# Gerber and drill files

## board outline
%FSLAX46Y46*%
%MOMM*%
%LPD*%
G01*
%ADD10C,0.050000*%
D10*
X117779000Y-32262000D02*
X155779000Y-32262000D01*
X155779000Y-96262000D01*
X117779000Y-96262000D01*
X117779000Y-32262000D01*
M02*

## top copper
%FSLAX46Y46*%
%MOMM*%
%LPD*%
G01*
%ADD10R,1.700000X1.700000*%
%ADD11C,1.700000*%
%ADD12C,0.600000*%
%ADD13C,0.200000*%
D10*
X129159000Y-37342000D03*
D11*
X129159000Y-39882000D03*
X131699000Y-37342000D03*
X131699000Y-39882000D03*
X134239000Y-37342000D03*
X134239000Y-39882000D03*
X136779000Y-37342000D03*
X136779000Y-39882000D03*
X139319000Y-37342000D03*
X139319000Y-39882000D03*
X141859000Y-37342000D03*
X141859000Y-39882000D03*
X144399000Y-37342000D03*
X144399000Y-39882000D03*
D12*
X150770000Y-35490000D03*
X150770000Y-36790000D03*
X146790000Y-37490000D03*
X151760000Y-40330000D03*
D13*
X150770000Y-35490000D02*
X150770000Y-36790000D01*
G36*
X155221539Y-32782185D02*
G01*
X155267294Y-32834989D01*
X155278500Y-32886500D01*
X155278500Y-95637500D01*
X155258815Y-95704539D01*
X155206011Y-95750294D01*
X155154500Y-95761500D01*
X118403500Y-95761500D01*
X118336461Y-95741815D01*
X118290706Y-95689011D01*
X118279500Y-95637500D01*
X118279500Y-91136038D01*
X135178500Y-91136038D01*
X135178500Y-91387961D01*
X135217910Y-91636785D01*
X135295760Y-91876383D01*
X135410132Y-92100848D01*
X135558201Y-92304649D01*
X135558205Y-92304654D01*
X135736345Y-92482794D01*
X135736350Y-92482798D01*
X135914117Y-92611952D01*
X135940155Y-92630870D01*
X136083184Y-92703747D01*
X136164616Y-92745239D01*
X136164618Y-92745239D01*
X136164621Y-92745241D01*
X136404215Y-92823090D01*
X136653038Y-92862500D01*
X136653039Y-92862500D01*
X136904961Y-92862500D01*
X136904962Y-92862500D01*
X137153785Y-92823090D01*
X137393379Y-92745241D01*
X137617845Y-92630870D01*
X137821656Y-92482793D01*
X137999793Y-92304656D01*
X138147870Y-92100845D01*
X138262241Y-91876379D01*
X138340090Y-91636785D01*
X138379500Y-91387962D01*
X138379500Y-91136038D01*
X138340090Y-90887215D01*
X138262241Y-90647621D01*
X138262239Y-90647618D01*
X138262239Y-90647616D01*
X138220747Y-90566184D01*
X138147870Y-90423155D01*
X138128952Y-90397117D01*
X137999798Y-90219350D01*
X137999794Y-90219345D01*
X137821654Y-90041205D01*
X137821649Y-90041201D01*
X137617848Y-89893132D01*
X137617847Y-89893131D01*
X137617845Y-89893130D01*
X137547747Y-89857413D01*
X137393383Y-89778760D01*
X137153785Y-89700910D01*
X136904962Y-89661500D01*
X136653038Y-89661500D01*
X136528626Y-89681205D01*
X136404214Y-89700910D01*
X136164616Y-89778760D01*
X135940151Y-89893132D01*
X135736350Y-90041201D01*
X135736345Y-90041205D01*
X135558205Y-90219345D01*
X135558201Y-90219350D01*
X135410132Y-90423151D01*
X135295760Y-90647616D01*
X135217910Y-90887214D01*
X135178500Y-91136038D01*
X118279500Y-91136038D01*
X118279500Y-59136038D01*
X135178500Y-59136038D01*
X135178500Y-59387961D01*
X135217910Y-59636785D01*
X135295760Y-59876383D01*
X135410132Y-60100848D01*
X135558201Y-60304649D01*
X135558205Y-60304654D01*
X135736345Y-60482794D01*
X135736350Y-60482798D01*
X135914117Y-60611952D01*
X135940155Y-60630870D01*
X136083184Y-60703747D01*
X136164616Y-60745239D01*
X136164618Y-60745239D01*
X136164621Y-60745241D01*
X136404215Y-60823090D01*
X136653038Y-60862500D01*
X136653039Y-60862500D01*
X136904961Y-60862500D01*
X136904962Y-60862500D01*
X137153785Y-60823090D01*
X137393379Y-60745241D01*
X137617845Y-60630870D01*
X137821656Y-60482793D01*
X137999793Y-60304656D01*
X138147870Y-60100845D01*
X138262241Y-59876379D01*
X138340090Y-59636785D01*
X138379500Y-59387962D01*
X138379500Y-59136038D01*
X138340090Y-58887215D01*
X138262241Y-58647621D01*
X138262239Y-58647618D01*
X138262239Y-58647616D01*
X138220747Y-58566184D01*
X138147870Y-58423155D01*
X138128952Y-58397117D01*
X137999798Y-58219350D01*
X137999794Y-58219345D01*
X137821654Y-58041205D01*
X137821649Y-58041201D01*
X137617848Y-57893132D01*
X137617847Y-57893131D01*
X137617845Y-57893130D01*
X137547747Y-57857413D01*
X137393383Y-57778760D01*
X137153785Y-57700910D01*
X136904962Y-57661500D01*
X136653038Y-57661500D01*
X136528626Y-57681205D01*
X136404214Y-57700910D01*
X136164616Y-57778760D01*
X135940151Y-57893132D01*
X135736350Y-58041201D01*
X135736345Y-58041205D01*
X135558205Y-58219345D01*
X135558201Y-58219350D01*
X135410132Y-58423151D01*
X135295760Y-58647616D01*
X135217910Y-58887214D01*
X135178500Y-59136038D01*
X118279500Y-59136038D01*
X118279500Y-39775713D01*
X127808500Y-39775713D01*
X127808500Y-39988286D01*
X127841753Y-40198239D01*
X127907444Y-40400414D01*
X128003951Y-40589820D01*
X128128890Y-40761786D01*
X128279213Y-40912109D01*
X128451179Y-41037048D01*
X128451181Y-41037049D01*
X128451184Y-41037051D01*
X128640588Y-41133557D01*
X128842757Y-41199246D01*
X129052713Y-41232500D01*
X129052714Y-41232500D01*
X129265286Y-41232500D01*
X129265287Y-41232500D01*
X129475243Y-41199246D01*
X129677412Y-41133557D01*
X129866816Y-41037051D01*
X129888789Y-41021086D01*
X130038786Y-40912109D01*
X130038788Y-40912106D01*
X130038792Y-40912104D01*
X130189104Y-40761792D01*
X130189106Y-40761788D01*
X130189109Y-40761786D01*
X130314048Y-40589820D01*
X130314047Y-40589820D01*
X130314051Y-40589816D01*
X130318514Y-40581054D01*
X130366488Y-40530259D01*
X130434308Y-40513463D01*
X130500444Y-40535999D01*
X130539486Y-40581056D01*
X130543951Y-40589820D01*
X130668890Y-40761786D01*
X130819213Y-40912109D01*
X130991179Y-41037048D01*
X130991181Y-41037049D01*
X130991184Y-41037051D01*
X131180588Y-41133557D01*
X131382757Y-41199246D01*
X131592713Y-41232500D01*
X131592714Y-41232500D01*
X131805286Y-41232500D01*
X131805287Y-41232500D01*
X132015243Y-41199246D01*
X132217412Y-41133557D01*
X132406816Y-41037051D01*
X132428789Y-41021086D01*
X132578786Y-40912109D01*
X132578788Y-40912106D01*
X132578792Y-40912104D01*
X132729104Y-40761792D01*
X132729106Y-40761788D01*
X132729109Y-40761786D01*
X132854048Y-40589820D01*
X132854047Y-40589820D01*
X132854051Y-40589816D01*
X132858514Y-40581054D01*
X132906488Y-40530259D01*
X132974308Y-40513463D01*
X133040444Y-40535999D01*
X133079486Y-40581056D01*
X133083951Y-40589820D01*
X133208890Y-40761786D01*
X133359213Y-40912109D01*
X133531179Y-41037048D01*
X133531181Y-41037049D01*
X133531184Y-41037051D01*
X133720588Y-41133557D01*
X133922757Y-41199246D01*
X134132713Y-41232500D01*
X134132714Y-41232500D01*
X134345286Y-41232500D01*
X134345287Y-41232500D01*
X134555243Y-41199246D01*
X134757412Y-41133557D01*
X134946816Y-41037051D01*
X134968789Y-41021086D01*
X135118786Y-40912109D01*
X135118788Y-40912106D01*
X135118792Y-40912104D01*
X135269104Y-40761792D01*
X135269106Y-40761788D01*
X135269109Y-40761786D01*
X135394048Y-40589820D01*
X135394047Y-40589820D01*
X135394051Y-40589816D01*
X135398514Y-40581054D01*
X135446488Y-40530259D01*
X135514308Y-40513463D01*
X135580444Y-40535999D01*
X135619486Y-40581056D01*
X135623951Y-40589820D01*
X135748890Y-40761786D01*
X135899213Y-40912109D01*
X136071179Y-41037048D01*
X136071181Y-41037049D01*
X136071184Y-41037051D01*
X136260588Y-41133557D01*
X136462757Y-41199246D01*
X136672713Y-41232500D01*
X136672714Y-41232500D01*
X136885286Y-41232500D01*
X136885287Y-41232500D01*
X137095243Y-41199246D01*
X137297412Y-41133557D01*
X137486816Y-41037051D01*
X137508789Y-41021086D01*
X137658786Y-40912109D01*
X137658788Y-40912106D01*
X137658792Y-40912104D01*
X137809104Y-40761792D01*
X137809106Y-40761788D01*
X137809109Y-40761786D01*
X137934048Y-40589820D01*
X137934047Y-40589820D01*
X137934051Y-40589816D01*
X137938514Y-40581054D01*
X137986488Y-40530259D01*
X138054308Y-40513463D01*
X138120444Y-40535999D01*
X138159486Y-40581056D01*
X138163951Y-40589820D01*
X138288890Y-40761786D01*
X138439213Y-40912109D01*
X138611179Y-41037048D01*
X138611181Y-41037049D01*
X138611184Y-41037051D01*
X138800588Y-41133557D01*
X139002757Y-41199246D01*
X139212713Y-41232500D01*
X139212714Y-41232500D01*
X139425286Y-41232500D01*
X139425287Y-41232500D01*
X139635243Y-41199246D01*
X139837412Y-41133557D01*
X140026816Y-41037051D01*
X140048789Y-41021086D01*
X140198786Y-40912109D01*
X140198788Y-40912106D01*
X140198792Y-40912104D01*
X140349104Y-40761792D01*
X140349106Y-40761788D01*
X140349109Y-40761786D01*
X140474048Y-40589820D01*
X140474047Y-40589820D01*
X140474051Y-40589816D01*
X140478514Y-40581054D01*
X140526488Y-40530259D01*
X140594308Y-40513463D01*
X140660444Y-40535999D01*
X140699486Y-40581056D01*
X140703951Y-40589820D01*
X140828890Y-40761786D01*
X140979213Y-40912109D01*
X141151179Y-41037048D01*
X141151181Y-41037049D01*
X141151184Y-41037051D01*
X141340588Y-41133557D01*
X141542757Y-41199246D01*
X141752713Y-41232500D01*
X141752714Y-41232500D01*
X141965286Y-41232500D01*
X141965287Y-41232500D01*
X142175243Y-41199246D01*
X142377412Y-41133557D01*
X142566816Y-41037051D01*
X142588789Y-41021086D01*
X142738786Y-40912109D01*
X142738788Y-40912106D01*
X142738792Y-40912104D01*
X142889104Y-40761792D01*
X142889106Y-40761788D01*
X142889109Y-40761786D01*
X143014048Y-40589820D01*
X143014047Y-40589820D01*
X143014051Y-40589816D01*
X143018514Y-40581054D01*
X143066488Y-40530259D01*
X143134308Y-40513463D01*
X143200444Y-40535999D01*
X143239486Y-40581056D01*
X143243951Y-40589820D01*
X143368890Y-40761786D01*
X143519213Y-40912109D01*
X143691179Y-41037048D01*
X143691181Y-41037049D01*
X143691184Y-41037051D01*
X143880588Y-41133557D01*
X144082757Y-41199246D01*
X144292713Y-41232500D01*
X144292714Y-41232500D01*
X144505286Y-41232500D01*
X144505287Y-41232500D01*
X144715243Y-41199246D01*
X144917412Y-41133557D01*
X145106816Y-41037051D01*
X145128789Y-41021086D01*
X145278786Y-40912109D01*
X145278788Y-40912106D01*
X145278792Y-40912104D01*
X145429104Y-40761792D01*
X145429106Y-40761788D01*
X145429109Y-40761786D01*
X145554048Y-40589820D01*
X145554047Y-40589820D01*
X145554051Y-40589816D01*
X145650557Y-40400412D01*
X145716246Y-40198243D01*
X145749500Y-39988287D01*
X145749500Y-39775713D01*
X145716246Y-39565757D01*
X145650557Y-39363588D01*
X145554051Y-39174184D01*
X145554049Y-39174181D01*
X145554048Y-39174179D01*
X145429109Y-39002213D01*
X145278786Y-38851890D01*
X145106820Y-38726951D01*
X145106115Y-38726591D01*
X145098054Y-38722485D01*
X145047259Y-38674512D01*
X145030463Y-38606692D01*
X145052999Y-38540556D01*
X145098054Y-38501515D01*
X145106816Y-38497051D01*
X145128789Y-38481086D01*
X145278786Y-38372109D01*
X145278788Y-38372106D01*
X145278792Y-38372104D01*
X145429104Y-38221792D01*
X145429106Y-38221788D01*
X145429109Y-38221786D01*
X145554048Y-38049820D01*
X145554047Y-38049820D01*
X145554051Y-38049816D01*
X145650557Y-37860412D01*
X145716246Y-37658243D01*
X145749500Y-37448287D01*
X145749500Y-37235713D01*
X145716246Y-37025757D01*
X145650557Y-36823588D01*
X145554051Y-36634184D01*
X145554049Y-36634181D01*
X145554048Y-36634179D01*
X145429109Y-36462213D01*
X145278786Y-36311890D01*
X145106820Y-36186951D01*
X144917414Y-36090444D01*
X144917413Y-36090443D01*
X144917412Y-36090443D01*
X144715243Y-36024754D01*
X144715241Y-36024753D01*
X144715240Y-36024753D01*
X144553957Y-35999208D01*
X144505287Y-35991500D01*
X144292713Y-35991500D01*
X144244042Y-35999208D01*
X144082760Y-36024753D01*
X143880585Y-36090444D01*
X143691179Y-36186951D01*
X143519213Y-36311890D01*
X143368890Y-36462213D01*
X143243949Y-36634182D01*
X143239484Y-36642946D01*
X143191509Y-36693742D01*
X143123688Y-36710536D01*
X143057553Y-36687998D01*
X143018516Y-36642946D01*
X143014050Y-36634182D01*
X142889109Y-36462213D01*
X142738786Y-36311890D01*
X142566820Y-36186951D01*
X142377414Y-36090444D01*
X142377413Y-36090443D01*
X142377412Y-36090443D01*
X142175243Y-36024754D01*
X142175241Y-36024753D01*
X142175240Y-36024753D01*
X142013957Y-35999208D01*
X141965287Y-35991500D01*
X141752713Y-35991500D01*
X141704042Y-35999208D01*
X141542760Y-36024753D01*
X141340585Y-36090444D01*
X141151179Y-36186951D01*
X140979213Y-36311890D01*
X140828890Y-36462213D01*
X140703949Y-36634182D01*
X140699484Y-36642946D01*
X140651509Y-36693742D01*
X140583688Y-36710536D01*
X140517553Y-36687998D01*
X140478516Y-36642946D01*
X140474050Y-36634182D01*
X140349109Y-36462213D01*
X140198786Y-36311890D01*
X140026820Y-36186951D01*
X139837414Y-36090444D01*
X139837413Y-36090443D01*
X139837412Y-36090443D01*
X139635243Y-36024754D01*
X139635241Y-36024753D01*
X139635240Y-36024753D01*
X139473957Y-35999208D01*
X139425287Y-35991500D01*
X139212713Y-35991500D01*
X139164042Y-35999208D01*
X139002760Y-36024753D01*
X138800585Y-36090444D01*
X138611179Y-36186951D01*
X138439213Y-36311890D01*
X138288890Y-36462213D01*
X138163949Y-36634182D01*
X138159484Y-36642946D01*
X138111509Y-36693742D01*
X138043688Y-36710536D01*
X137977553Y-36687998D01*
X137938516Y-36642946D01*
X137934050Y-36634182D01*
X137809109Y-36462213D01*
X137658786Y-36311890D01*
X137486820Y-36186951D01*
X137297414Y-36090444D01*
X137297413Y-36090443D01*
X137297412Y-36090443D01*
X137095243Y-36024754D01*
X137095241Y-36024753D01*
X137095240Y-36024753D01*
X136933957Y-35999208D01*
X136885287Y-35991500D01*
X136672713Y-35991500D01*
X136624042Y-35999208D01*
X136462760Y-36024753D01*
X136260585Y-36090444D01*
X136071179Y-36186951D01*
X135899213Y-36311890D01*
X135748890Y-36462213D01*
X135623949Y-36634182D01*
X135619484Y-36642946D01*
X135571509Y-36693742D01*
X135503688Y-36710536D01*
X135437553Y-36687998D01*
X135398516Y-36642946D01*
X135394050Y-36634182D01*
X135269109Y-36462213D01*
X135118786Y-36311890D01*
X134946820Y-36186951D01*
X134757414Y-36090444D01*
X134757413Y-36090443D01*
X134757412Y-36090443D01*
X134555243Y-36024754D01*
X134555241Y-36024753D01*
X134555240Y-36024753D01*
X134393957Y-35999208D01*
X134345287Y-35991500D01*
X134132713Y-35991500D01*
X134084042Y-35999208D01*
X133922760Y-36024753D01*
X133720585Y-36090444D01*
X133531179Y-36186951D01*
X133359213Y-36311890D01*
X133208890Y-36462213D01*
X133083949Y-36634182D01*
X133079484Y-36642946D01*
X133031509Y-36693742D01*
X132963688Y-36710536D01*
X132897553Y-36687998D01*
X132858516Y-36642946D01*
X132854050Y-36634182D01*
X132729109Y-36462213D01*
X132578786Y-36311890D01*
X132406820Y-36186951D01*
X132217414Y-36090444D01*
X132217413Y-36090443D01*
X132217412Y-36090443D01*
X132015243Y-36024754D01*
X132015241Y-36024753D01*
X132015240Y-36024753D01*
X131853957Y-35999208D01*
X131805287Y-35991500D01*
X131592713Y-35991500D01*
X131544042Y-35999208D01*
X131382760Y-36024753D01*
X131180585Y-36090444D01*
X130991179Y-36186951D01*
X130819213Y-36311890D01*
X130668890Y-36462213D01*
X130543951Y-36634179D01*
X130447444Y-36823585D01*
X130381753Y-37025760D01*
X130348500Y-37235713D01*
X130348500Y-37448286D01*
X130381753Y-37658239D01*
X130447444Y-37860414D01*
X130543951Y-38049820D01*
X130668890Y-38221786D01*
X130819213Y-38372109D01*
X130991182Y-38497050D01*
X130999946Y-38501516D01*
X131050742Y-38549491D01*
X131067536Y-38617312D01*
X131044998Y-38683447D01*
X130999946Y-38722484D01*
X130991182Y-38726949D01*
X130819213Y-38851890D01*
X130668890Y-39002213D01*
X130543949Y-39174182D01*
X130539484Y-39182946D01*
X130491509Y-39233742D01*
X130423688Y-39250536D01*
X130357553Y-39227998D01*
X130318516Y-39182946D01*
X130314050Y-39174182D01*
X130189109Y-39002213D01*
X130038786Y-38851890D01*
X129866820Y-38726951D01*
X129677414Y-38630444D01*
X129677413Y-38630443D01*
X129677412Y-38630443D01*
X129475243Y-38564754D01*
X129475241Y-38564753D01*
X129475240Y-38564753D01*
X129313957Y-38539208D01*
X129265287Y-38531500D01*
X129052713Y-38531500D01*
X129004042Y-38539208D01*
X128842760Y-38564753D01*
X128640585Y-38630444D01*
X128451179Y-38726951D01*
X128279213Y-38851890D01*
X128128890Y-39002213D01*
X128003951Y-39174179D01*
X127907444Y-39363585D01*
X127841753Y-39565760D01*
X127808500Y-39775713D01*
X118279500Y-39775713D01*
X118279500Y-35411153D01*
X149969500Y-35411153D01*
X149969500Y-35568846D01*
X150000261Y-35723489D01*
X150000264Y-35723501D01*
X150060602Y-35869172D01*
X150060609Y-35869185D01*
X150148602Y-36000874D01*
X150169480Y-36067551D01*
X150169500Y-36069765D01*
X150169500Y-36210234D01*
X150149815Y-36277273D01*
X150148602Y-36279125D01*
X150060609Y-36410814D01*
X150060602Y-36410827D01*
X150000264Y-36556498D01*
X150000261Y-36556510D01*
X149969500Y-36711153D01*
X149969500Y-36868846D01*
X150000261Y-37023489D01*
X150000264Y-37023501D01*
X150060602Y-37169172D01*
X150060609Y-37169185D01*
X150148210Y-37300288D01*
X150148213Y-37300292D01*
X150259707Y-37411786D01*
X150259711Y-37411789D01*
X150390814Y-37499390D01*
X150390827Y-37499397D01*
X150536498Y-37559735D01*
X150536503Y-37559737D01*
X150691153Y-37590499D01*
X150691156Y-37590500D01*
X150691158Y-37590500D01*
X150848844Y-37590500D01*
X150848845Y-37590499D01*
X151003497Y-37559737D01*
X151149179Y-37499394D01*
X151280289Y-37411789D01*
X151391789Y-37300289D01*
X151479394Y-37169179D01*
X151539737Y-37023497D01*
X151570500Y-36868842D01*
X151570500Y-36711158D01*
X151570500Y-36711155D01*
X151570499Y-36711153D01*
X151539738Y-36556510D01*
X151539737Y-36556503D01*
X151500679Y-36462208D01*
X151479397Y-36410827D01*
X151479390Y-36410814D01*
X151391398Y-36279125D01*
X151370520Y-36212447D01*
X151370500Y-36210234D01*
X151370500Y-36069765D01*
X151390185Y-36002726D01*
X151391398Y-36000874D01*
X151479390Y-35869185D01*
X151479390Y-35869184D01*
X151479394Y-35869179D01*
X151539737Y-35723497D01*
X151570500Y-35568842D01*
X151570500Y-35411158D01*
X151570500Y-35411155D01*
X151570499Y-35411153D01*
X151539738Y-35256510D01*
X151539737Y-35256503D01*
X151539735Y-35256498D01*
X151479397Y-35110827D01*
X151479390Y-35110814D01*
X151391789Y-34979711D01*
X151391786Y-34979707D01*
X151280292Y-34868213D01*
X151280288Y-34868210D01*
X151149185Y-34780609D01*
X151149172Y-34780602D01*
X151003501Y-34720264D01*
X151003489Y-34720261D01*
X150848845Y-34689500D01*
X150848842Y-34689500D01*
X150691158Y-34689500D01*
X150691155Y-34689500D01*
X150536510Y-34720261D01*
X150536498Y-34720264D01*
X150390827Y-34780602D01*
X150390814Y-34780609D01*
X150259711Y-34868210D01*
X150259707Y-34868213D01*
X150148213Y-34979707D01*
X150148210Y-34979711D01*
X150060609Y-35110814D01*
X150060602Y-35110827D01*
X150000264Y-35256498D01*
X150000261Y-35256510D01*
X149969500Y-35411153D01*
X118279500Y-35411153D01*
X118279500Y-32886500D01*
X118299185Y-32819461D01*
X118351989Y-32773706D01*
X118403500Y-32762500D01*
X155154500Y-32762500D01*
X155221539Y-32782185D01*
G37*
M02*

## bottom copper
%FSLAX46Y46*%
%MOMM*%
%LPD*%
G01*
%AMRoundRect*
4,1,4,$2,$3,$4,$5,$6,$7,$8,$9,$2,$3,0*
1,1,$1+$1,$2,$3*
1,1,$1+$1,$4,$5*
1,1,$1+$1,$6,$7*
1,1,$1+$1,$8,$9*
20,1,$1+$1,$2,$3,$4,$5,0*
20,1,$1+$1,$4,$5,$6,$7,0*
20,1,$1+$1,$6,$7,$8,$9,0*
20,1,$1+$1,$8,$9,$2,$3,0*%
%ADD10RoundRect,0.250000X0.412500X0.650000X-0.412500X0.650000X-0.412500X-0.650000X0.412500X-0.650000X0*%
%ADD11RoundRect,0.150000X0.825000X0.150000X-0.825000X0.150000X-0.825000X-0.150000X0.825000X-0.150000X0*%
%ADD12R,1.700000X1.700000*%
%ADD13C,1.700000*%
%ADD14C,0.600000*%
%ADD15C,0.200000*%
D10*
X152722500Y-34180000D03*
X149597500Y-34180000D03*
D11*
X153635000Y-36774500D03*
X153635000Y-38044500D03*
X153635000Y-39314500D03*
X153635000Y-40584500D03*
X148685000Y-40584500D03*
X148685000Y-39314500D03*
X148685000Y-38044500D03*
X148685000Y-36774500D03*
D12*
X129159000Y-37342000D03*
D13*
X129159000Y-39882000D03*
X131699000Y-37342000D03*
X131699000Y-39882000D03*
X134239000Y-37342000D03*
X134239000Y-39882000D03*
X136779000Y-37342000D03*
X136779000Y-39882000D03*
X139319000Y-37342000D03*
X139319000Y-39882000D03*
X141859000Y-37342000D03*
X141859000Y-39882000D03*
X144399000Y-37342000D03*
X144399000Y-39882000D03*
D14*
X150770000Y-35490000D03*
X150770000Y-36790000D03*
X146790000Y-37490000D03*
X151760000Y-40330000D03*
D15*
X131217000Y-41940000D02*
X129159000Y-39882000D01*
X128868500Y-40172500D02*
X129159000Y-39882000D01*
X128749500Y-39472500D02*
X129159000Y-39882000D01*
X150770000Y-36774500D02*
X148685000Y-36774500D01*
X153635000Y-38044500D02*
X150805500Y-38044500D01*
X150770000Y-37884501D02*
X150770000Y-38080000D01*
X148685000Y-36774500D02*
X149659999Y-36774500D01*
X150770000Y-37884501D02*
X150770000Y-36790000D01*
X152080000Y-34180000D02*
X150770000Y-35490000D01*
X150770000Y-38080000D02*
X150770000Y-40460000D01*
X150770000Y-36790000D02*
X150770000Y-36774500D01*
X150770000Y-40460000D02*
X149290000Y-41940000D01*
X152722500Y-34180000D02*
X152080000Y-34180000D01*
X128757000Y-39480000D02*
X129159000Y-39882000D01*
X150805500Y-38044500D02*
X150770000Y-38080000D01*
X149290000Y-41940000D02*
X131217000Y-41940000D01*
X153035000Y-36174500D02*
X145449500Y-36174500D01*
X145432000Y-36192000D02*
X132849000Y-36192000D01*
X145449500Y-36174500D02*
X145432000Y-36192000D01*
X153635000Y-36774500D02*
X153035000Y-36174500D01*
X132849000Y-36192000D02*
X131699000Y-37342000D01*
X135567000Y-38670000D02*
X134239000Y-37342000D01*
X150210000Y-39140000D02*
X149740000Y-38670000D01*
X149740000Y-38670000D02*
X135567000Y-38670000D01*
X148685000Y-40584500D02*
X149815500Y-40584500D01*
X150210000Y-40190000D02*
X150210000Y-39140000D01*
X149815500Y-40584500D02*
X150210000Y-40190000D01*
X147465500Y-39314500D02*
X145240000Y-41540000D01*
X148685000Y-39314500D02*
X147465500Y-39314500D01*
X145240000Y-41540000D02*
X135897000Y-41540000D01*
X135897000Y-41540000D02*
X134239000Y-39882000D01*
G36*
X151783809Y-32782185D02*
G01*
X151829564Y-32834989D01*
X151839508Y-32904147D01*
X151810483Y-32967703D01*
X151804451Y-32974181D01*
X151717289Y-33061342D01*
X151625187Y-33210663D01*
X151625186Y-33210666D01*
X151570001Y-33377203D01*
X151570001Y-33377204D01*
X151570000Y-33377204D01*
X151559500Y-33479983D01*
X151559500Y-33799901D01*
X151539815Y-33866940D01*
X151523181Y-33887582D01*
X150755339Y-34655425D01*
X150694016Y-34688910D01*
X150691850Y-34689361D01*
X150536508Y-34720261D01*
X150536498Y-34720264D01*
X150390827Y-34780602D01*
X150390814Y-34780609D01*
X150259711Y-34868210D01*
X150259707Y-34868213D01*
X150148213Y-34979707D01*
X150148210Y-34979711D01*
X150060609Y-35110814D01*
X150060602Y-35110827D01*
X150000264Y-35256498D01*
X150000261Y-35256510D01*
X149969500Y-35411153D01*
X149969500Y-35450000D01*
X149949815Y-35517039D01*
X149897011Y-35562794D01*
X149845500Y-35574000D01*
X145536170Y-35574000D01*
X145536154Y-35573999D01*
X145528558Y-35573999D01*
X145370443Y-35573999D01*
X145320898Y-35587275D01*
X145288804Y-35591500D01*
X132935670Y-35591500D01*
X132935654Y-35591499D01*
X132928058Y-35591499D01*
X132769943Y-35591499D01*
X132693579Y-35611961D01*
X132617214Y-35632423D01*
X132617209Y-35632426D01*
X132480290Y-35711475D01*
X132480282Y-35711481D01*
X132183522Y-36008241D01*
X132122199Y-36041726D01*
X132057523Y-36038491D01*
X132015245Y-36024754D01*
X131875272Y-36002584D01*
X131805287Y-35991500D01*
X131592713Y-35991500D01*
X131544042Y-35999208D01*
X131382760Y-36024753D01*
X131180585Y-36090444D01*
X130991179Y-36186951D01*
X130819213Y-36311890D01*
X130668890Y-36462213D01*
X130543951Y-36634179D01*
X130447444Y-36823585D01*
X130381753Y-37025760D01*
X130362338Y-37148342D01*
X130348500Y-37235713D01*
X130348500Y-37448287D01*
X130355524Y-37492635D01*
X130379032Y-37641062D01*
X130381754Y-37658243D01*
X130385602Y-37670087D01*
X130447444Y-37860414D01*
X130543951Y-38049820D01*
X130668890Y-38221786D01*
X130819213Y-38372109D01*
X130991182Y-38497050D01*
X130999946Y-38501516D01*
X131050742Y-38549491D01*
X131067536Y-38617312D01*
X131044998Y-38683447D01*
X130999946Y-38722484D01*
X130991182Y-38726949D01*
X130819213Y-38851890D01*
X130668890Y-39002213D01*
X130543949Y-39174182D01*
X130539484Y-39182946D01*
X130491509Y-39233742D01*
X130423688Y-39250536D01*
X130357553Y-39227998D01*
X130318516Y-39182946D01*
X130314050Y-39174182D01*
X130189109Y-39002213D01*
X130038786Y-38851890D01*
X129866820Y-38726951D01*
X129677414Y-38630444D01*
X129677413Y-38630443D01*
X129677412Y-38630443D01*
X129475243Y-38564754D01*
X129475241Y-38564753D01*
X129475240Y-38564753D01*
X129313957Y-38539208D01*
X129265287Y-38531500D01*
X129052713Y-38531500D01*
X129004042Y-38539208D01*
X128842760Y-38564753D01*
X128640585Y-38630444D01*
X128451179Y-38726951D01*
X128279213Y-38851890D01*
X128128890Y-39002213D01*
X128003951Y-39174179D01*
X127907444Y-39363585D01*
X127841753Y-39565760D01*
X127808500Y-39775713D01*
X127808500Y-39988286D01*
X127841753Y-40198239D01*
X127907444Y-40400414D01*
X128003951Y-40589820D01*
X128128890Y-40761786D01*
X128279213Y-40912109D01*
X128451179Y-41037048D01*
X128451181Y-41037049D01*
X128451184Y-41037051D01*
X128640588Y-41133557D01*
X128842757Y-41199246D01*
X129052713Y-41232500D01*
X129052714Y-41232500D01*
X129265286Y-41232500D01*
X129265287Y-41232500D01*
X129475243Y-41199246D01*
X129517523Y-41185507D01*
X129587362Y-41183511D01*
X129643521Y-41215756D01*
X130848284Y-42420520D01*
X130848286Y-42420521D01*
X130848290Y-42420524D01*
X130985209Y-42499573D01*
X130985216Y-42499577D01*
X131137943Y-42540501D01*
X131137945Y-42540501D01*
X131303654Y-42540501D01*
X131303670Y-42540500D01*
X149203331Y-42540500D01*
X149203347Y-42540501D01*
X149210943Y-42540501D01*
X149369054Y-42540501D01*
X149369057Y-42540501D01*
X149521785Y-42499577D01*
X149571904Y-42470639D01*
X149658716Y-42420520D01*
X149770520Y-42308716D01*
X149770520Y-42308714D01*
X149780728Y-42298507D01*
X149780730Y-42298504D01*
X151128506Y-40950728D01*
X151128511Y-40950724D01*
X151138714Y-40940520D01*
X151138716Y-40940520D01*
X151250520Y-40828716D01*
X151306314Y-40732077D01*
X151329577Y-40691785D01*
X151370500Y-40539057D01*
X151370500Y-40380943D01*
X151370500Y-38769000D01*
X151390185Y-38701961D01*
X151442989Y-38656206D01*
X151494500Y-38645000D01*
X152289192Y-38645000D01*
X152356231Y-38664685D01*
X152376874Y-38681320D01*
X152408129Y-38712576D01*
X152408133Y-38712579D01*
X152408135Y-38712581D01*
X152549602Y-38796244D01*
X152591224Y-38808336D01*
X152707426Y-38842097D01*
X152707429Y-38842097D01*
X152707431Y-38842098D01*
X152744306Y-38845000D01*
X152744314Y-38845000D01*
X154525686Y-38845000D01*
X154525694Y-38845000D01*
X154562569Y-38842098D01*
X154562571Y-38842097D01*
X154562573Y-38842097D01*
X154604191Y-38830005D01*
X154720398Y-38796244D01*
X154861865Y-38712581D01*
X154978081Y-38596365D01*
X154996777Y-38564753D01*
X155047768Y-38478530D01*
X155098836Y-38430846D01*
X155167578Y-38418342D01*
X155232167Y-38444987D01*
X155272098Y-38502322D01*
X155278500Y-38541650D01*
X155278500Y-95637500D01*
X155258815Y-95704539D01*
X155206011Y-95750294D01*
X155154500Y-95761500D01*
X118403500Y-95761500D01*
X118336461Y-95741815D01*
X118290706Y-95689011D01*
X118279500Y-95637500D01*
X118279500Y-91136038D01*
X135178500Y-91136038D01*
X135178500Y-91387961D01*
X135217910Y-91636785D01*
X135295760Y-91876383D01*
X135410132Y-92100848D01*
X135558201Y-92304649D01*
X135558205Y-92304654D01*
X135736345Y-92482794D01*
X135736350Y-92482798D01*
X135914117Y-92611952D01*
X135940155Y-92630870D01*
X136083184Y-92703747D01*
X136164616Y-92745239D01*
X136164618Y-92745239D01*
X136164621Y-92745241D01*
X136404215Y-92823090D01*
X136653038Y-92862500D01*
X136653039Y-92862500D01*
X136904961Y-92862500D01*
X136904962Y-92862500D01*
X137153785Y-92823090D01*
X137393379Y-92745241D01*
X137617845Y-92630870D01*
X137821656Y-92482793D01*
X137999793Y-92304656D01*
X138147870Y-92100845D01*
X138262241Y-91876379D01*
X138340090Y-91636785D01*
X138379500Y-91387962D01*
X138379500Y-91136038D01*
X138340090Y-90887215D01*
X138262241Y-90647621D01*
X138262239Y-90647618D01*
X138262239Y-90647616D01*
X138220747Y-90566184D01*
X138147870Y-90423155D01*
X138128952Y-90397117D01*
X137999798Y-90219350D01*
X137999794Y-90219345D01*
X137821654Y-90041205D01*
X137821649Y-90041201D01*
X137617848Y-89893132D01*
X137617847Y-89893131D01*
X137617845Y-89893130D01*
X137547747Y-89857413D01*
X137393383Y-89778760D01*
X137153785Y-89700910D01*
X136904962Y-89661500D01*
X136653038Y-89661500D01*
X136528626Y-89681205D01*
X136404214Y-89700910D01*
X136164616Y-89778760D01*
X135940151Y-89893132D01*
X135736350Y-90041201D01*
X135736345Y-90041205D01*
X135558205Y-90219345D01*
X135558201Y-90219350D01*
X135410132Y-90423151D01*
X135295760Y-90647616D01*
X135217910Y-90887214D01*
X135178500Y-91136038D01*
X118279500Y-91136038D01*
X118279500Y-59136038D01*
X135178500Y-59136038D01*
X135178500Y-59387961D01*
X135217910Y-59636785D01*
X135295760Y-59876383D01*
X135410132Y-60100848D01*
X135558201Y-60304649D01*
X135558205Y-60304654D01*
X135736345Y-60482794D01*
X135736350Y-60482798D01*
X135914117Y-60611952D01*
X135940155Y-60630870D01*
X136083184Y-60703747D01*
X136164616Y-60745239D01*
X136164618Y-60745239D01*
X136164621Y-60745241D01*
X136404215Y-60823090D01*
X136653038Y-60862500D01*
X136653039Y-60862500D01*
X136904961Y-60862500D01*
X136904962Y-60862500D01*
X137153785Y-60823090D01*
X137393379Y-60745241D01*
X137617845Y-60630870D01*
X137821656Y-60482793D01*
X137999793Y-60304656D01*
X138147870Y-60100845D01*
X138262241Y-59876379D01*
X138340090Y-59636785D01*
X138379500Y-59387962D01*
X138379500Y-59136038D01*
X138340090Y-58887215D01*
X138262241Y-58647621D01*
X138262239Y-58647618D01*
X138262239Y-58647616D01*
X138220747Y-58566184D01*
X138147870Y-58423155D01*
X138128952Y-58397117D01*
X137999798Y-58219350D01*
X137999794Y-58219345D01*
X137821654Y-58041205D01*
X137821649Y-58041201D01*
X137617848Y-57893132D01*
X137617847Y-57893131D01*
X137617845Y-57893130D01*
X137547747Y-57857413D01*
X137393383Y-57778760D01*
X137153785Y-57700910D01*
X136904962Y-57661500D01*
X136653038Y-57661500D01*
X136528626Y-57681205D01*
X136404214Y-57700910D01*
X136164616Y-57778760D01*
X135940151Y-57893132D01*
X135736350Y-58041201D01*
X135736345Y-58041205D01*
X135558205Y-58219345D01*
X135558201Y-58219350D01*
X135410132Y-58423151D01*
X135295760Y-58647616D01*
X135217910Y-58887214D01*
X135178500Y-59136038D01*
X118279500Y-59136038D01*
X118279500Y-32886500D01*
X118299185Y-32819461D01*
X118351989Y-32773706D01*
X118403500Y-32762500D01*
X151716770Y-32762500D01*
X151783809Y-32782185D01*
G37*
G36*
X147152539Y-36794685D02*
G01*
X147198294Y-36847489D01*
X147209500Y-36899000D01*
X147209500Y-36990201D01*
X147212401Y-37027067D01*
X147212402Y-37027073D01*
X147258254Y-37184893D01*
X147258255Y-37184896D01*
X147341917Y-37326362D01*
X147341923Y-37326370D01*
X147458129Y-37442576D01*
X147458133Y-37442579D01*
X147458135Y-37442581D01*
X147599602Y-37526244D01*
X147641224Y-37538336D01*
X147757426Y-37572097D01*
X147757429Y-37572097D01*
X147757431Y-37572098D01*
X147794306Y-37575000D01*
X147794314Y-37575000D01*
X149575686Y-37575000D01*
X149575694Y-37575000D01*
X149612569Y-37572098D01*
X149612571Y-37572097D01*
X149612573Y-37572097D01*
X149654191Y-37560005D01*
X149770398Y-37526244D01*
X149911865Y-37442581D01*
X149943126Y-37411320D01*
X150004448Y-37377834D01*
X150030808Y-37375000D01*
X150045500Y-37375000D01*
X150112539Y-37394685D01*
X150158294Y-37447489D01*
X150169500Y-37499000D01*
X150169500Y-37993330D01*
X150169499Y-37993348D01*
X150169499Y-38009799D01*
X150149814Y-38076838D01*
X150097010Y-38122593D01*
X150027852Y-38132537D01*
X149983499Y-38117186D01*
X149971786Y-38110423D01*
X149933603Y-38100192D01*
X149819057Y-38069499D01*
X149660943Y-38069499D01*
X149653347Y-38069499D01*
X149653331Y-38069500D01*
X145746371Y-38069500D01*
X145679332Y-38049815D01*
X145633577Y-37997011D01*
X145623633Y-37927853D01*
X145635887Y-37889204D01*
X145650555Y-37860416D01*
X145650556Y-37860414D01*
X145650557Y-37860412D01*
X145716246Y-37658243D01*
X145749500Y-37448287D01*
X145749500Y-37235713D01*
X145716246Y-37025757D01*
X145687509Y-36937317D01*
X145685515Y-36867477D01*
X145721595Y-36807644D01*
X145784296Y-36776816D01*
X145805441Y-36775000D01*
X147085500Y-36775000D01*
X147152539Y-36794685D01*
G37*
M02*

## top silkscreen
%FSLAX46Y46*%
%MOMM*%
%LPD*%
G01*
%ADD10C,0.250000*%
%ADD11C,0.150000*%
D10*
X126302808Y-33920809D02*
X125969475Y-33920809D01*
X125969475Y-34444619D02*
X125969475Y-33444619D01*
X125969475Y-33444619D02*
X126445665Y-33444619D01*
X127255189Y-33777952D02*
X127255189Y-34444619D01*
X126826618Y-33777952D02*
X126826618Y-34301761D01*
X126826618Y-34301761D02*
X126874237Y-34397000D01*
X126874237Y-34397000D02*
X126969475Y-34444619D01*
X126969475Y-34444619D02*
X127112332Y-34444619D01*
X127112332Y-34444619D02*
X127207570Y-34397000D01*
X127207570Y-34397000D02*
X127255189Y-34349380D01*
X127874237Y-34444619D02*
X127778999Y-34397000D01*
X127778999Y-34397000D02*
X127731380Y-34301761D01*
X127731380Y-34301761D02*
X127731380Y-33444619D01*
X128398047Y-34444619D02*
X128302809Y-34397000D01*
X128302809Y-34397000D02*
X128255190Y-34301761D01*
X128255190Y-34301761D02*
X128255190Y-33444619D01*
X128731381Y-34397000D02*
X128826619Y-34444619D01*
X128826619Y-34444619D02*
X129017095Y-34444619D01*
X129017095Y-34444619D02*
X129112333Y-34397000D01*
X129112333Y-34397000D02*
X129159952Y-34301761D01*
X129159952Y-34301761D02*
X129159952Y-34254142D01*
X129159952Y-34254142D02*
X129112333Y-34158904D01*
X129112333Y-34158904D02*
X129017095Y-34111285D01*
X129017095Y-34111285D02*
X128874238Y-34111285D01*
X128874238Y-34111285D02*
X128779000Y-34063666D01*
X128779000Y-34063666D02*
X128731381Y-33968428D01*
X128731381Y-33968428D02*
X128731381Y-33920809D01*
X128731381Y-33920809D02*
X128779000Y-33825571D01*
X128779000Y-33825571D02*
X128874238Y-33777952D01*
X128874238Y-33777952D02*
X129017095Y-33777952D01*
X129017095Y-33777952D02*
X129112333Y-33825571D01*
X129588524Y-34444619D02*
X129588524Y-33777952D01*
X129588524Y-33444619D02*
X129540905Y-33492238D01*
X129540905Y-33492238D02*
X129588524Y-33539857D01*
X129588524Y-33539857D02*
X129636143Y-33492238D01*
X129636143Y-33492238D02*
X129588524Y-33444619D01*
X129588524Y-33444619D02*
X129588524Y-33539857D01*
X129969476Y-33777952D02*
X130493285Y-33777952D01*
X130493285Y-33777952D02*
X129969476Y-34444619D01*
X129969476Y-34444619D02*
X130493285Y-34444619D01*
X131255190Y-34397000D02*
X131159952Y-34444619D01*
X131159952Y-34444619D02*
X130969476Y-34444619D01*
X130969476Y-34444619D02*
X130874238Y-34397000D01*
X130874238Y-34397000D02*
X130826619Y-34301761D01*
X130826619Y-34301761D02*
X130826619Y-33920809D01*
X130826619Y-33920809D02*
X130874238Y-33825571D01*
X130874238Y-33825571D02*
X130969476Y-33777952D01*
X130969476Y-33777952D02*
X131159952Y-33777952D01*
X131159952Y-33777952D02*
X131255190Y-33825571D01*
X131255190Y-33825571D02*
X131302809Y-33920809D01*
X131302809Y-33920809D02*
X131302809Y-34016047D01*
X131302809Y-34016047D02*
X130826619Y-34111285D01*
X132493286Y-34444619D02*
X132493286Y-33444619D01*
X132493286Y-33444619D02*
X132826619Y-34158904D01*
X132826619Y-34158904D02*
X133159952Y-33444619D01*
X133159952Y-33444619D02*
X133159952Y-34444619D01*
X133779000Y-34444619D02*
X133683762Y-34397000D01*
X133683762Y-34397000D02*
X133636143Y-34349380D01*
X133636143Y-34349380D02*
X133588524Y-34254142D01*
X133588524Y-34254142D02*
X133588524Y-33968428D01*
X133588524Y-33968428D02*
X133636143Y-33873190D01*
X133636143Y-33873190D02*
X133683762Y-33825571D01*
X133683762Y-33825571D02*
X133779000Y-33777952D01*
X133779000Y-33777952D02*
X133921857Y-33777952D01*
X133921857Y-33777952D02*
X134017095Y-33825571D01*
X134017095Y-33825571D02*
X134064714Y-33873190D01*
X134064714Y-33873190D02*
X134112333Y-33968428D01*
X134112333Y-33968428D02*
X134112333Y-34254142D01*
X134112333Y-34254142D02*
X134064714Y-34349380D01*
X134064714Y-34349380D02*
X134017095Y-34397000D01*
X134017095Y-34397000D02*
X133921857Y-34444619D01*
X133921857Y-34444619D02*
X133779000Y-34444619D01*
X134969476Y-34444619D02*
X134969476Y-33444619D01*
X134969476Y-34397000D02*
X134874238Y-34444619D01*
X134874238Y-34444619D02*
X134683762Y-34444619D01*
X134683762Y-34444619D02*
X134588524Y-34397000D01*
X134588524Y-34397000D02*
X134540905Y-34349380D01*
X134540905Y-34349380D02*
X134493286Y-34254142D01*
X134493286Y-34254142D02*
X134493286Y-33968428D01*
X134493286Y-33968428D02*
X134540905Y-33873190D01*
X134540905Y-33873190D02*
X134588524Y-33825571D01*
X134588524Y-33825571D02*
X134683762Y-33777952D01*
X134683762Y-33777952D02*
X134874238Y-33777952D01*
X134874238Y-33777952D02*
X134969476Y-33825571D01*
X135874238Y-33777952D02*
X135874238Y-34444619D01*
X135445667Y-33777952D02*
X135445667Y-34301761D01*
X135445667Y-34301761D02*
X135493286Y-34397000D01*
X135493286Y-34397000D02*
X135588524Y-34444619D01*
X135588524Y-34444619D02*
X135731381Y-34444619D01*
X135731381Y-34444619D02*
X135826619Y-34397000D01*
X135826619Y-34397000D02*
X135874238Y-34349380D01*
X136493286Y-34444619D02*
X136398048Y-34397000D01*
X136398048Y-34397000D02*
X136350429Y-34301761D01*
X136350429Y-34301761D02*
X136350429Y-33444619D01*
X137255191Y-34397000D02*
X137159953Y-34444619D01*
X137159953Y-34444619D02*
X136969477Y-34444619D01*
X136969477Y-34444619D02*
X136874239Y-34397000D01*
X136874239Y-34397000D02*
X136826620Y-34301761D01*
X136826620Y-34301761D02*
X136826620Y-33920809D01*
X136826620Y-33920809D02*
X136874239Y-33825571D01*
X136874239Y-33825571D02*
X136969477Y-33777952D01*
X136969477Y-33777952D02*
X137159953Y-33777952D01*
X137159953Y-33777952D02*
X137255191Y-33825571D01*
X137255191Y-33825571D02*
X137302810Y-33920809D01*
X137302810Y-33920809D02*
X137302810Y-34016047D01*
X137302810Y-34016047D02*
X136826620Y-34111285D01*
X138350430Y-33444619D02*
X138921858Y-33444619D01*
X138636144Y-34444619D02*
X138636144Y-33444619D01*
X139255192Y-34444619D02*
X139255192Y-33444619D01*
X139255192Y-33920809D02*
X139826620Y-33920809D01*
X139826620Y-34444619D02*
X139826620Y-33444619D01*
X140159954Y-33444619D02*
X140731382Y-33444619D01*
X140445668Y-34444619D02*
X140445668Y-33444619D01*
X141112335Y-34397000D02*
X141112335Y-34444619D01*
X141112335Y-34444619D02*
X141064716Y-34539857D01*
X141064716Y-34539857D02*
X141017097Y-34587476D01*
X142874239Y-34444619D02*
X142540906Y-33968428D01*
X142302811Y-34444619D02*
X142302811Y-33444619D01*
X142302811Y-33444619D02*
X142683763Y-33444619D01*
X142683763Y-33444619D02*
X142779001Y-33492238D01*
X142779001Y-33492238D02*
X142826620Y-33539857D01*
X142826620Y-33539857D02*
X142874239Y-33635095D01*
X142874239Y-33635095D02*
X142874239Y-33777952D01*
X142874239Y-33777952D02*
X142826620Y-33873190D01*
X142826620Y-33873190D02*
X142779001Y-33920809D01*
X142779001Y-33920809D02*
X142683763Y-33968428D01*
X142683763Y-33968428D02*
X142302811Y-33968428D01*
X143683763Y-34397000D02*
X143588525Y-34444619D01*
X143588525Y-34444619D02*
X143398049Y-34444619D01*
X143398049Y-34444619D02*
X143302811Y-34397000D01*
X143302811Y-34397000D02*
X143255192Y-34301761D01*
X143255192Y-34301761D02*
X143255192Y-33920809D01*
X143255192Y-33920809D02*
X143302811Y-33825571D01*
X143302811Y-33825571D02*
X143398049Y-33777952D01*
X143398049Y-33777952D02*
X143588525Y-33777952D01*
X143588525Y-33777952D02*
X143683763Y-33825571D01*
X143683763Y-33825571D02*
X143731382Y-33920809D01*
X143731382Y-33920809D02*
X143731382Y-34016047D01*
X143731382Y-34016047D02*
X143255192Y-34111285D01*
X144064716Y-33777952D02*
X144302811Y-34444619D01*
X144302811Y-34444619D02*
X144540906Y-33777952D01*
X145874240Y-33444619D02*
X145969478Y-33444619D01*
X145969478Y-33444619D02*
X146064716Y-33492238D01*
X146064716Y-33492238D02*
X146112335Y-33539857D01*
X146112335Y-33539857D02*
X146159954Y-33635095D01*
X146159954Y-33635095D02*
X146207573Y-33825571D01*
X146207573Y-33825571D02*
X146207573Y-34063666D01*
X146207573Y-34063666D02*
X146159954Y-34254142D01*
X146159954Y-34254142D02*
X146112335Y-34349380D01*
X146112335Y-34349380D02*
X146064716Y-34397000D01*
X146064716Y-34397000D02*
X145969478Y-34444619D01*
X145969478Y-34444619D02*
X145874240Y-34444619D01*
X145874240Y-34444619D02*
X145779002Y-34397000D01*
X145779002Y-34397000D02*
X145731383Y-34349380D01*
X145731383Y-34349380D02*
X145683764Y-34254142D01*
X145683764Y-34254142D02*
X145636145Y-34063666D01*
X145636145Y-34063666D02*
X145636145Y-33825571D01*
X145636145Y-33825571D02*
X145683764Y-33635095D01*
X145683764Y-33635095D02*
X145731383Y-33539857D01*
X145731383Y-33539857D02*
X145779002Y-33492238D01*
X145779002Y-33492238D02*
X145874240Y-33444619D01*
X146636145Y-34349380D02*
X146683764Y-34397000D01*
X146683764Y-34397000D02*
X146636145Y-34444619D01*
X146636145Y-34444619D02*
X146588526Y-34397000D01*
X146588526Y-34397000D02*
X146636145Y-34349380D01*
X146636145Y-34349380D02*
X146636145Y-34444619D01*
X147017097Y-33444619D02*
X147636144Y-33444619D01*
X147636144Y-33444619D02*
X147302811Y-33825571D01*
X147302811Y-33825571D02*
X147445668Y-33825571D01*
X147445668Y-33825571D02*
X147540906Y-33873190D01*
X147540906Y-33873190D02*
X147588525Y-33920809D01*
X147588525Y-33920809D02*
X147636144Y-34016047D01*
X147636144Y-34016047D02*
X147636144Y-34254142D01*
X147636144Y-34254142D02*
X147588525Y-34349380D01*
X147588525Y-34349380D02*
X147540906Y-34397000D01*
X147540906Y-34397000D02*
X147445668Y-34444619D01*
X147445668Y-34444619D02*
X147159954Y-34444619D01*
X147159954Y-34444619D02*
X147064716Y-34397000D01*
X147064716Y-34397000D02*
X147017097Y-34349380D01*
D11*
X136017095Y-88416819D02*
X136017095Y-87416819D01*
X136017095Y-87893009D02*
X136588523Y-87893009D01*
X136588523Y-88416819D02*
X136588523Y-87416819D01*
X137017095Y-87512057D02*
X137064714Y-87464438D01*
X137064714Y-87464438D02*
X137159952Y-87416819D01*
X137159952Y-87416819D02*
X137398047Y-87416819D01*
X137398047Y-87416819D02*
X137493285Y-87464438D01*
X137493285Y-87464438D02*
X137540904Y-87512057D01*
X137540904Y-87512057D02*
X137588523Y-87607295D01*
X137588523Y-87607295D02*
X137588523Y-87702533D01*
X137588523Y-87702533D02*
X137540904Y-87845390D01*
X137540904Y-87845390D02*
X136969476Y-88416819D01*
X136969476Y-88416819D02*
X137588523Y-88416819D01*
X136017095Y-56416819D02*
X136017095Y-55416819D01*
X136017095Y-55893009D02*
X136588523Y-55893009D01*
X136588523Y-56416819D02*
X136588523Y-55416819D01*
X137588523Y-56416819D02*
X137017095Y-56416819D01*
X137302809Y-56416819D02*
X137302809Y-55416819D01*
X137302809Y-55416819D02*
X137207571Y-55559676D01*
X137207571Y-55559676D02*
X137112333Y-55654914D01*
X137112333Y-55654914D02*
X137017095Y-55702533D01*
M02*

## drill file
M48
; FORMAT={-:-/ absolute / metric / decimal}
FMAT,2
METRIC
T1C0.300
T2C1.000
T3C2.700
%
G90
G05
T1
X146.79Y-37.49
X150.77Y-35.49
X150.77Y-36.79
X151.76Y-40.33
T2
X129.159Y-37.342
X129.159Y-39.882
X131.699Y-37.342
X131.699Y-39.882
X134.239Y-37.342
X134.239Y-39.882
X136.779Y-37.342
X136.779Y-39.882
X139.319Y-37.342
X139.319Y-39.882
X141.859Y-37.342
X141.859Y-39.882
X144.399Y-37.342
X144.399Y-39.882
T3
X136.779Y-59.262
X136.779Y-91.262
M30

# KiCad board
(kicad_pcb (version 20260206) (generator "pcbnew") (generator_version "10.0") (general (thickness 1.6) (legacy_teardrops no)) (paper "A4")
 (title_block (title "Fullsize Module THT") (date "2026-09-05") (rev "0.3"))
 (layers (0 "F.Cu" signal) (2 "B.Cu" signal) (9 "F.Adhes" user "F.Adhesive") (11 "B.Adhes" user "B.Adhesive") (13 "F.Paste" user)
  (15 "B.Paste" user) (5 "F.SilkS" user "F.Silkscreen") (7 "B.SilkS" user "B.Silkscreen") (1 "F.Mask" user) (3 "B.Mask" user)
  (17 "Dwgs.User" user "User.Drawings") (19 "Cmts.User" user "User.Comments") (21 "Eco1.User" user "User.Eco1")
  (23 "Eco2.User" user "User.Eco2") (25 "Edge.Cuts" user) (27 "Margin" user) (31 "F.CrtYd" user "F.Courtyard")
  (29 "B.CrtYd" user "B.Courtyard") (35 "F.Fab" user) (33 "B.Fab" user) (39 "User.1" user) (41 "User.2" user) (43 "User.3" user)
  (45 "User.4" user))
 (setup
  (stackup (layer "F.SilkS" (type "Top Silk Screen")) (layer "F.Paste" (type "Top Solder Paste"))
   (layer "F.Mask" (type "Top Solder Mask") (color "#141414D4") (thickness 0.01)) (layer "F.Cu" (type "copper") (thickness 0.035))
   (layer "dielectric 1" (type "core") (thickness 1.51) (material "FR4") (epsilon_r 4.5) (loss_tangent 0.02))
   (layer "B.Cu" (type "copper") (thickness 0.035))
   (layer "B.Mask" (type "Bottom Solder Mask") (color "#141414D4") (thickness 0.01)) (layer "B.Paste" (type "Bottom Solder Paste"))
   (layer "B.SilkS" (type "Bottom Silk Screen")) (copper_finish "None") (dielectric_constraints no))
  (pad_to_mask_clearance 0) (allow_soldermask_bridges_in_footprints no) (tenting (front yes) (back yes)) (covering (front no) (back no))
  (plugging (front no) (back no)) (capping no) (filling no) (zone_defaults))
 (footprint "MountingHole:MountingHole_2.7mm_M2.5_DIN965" (layer "F.Cu") (at 136.779 91.262)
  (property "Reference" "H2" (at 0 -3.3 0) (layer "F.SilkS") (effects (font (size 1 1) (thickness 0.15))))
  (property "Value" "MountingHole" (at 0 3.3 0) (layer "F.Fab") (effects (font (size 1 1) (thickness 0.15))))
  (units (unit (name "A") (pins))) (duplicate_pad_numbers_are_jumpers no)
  (pad "" np_thru_hole circle (at 0 0) (size 2.7 2.7) (drill 2.7) (layers "*.Cu" "*.Mask")))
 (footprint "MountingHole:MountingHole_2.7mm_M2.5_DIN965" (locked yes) (layer "F.Cu") (at 136.779 59.262)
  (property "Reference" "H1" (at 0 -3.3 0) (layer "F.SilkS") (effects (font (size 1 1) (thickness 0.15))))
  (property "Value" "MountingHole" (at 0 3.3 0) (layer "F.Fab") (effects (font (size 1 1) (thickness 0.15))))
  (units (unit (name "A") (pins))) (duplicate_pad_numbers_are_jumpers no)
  (pad "" np_thru_hole circle (at 0 0) (size 2.7 2.7) (drill 2.7) (layers "*.Cu" "*.Mask")))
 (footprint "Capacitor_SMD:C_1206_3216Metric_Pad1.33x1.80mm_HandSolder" (layer "B.Cu") (at 151.16 34.18 180)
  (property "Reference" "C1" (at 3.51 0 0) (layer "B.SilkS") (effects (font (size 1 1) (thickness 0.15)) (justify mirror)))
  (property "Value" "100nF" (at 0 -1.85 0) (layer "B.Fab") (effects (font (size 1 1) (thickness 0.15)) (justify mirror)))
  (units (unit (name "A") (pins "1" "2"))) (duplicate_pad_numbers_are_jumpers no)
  (pad "1" smd roundrect (at -1.5625 0 180) (size 1.325 1.8) (layers "B.Cu" "B.Mask" "B.Paste") (roundrect_rratio 0.188679) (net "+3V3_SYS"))
  (pad "2" smd roundrect (at 1.5625 0 180) (size 1.325 1.8) (layers "B.Cu" "B.Mask" "B.Paste") (roundrect_rratio 0.188679) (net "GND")
   (zone_connect 2)))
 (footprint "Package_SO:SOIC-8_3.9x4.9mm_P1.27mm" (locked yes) (layer "B.Cu") (at 151.16 38.6795 180)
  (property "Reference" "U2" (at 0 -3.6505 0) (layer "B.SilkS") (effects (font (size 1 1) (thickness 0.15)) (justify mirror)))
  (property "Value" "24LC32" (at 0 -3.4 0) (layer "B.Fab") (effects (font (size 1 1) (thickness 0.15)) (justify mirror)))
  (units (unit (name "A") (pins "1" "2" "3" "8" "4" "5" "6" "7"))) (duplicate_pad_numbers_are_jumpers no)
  (pad "1" smd roundrect (at -2.475 1.905 180) (size 1.95 0.6) (layers "B.Cu" "B.Mask" "B.Paste") (roundrect_rratio 0.25) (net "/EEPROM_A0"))
  (pad "2" smd roundrect (at -2.475 0.635 180) (size 1.95 0.6) (layers "B.Cu" "B.Mask" "B.Paste") (roundrect_rratio 0.25) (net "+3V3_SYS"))
  (pad "3" smd roundrect (at -2.475 -0.635 180) (size 1.95 0.6) (layers "B.Cu" "B.Mask" "B.Paste") (roundrect_rratio 0.25) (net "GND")
   (zone_connect 2))
  (pad "4" smd roundrect (at -2.475 -1.905 180) (size 1.95 0.6) (layers "B.Cu" "B.Mask" "B.Paste") (roundrect_rratio 0.25) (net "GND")
   (zone_connect 2))
  (pad "5" smd roundrect (at 2.475 -1.905 180) (size 1.95 0.6) (layers "B.Cu" "B.Mask" "B.Paste") (roundrect_rratio 0.25) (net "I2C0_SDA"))
  (pad "6" smd roundrect (at 2.475 -0.635 180) (size 1.95 0.6) (layers "B.Cu" "B.Mask" "B.Paste") (roundrect_rratio 0.25) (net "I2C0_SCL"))
  (pad "7" smd roundrect (at 2.475 0.635 180) (size 1.95 0.6) (layers "B.Cu" "B.Mask" "B.Paste") (roundrect_rratio 0.25) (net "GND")
   (zone_connect 2))
  (pad "8" smd roundrect (at 2.475 1.905 180) (size 1.95 0.6) (layers "B.Cu" "B.Mask" "B.Paste") (roundrect_rratio 0.25) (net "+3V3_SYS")))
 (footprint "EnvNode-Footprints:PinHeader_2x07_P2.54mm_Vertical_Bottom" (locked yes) (layer "B.Cu") (at 129.159 37.342 -90)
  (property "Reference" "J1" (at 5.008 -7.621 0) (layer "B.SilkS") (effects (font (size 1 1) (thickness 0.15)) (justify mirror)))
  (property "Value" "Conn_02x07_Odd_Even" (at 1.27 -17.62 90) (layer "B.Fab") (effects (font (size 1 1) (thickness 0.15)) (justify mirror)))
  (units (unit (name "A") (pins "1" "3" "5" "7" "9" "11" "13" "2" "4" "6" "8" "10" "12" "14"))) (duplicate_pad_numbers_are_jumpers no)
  (pad "1" thru_hole rect (at 0 0 270) (size 1.7 1.7) (drill 1) (layers "*.Cu" "*.Mask") (remove_unused_layers no) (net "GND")
   (zone_connect 2))
  (pad "2" thru_hole circle (at 2.54 0 270) (size 1.7 1.7) (drill 1) (layers "*.Cu" "*.Mask") (remove_unused_layers no) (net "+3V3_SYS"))
  (pad "3" thru_hole circle (at 0 -2.54 270) (size 1.7 1.7) (drill 1) (layers "*.Cu" "*.Mask") (remove_unused_layers no) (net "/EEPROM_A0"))
  (pad "4" thru_hole circle (at 2.54 -2.54 270) (size 1.7 1.7) (drill 1) (layers "*.Cu" "*.Mask") (remove_unused_layers no) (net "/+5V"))
  (pad "5" thru_hole circle (at 0 -5.08 270) (size 1.7 1.7) (drill 1) (layers "*.Cu" "*.Mask") (remove_unused_layers no) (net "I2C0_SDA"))
  (pad "6" thru_hole circle (at 2.54 -5.08 270) (size 1.7 1.7) (drill 1) (layers "*.Cu" "*.Mask") (remove_unused_layers no) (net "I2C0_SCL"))
  (pad "7" thru_hole circle (at 0 -7.62 270) (size 1.7 1.7) (drill 1) (layers "*.Cu" "*.Mask") (remove_unused_layers no) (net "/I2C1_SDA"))
  (pad "8" thru_hole circle (at 2.54 -7.62 270) (size 1.7 1.7) (drill 1) (layers "*.Cu" "*.Mask") (remove_unused_layers no)
   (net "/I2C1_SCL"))
  (pad "9" thru_hole circle (at 0 -10.16 270) (size 1.7 1.7) (drill 1) (layers "*.Cu" "*.Mask") (remove_unused_layers no) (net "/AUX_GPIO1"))
  (pad "10" thru_hole circle (at 2.54 -10.16 270) (size 1.7 1.7) (drill 1) (layers "*.Cu" "*.Mask") (remove_unused_layers no)
   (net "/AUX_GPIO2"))
  (pad "11" thru_hole circle (at 0 -12.7 270) (size 1.7 1.7) (drill 1) (layers "*.Cu" "*.Mask") (remove_unused_layers no) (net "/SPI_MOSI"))
  (pad "12" thru_hole circle (at 2.54 -12.7 270) (size 1.7 1.7) (drill 1) (layers "*.Cu" "*.Mask") (remove_unused_layers no)
   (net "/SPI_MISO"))
  (pad "13" thru_hole circle (at 0 -15.24 270) (size 1.7 1.7) (drill 1) (layers "*.Cu" "*.Mask") (remove_unused_layers no) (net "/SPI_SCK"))
  (pad "14" thru_hole circle (at 2.54 -15.24 270) (size 1.7 1.7) (drill 1) (layers "*.Cu" "*.Mask") (remove_unused_layers no)
   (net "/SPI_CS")))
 (gr_rect (start 117.779 32.262) (end 155.779 96.262) (stroke (width 0.05) (type solid)) (fill no) (locked yes) (layer "Edge.Cuts"))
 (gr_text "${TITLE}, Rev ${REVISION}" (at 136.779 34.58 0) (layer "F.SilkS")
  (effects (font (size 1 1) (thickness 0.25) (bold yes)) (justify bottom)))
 (segment (start 150.77 35.49) (end 150.77 36.79) (width 0.2) (layer "F.Cu") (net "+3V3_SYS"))
 (via (at 150.77 35.49) (size 0.6) (drill 0.3) (layers "F.Cu" "B.Cu") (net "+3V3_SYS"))
 (via (at 150.77 36.79) (size 0.6) (drill 0.3) (layers "F.Cu" "B.Cu") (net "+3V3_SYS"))
 (segment (start 131.217 41.94) (end 129.159 39.882) (width 0.2) (layer "B.Cu") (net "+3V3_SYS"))
 (segment (start 128.8685 40.1725) (end 129.159 39.882) (width 0.2) (layer "B.Cu") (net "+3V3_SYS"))
 (segment (start 128.7495 39.4725) (end 129.159 39.882) (width 0.2) (layer "B.Cu") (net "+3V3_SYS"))
 (segment (start 150.77 36.7745) (end 148.685 36.7745) (width 0.2) (layer "B.Cu") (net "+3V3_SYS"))
 (segment (start 153.635 38.0445) (end 150.8055 38.0445) (width 0.2) (layer "B.Cu") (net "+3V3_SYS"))
 (segment (start 150.77 37.884501) (end 150.77 38.08) (width 0.2) (layer "B.Cu") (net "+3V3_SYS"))
 (segment (start 148.685 36.7745) (end 149.659999 36.7745) (width 0.2) (layer "B.Cu") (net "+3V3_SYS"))
 (segment (start 150.77 37.884501) (end 150.77 36.79) (width 0.2) (layer "B.Cu") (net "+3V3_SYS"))
 (segment (start 152.08 34.18) (end 150.77 35.49) (width 0.2) (layer "B.Cu") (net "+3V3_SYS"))
 (segment (start 150.77 38.08) (end 150.77 40.46) (width 0.2) (layer "B.Cu") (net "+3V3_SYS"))
 (segment (start 150.77 36.79) (end 150.77 36.7745) (width 0.2) (layer "B.Cu") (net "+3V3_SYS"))
 (segment (start 150.77 40.46) (end 149.29 41.94) (width 0.2) (layer "B.Cu") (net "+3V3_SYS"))
 (segment (start 152.7225 34.18) (end 152.08 34.18) (width 0.2) (layer "B.Cu") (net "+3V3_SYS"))
 (segment (start 128.757 39.48) (end 129.159 39.882) (width 0.2) (layer "B.Cu") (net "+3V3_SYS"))
 (segment (start 150.8055 38.0445) (end 150.77 38.08) (width 0.2) (layer "B.Cu") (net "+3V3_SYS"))
 (segment (start 149.29 41.94) (end 131.217 41.94) (width 0.2) (layer "B.Cu") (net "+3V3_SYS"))
 (via (at 146.79 37.49) (size 0.6) (drill 0.3) (layers "F.Cu" "B.Cu") (free yes) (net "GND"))
 (via (at 151.76 40.33) (size 0.6) (drill 0.3) (layers "F.Cu" "B.Cu") (free yes) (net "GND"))
 (segment (start 153.035 36.1745) (end 145.4495 36.1745) (width 0.2) (layer "B.Cu") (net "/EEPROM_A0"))
 (segment (start 145.432 36.192) (end 132.849 36.192) (width 0.2) (layer "B.Cu") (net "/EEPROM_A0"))
 (segment (start 145.4495 36.1745) (end 145.432 36.192) (width 0.2) (layer "B.Cu") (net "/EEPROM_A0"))
 (segment (start 153.635 36.7745) (end 153.035 36.1745) (width 0.2) (layer "B.Cu") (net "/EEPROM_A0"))
 (segment (start 132.849 36.192) (end 131.699 37.342) (width 0.2) (layer "B.Cu") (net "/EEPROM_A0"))
 (segment (start 135.567 38.67) (end 134.239 37.342) (width 0.2) (layer "B.Cu") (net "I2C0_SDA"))
 (segment (start 150.21 39.14) (end 149.74 38.67) (width 0.2) (layer "B.Cu") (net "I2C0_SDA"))
 (segment (start 149.74 38.67) (end 135.567 38.67) (width 0.2) (layer "B.Cu") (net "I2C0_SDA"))
 (segment (start 148.685 40.5845) (end 149.8155 40.5845) (width 0.2) (layer "B.Cu") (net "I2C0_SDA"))
 (segment (start 150.21 40.19) (end 150.21 39.14) (width 0.2) (layer "B.Cu") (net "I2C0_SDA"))
 (segment (start 149.8155 40.5845) (end 150.21 40.19) (width 0.2) (layer "B.Cu") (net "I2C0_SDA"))
 (segment (start 147.4655 39.3145) (end 145.24 41.54) (width 0.2) (layer "B.Cu") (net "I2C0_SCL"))
 (segment (start 148.685 39.3145) (end 147.4655 39.3145) (width 0.2) (layer "B.Cu") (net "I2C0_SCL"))
 (segment (start 145.24 41.54) (end 135.897 41.54) (width 0.2) (layer "B.Cu") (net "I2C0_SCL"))
 (segment (start 135.897 41.54) (end 134.239 39.882) (width 0.2) (layer "B.Cu") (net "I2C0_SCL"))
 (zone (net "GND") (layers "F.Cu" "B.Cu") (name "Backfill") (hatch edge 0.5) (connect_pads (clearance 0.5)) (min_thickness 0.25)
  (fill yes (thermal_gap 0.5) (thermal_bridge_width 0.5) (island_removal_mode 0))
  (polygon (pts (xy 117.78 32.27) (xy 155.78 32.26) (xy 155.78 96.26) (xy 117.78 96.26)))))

